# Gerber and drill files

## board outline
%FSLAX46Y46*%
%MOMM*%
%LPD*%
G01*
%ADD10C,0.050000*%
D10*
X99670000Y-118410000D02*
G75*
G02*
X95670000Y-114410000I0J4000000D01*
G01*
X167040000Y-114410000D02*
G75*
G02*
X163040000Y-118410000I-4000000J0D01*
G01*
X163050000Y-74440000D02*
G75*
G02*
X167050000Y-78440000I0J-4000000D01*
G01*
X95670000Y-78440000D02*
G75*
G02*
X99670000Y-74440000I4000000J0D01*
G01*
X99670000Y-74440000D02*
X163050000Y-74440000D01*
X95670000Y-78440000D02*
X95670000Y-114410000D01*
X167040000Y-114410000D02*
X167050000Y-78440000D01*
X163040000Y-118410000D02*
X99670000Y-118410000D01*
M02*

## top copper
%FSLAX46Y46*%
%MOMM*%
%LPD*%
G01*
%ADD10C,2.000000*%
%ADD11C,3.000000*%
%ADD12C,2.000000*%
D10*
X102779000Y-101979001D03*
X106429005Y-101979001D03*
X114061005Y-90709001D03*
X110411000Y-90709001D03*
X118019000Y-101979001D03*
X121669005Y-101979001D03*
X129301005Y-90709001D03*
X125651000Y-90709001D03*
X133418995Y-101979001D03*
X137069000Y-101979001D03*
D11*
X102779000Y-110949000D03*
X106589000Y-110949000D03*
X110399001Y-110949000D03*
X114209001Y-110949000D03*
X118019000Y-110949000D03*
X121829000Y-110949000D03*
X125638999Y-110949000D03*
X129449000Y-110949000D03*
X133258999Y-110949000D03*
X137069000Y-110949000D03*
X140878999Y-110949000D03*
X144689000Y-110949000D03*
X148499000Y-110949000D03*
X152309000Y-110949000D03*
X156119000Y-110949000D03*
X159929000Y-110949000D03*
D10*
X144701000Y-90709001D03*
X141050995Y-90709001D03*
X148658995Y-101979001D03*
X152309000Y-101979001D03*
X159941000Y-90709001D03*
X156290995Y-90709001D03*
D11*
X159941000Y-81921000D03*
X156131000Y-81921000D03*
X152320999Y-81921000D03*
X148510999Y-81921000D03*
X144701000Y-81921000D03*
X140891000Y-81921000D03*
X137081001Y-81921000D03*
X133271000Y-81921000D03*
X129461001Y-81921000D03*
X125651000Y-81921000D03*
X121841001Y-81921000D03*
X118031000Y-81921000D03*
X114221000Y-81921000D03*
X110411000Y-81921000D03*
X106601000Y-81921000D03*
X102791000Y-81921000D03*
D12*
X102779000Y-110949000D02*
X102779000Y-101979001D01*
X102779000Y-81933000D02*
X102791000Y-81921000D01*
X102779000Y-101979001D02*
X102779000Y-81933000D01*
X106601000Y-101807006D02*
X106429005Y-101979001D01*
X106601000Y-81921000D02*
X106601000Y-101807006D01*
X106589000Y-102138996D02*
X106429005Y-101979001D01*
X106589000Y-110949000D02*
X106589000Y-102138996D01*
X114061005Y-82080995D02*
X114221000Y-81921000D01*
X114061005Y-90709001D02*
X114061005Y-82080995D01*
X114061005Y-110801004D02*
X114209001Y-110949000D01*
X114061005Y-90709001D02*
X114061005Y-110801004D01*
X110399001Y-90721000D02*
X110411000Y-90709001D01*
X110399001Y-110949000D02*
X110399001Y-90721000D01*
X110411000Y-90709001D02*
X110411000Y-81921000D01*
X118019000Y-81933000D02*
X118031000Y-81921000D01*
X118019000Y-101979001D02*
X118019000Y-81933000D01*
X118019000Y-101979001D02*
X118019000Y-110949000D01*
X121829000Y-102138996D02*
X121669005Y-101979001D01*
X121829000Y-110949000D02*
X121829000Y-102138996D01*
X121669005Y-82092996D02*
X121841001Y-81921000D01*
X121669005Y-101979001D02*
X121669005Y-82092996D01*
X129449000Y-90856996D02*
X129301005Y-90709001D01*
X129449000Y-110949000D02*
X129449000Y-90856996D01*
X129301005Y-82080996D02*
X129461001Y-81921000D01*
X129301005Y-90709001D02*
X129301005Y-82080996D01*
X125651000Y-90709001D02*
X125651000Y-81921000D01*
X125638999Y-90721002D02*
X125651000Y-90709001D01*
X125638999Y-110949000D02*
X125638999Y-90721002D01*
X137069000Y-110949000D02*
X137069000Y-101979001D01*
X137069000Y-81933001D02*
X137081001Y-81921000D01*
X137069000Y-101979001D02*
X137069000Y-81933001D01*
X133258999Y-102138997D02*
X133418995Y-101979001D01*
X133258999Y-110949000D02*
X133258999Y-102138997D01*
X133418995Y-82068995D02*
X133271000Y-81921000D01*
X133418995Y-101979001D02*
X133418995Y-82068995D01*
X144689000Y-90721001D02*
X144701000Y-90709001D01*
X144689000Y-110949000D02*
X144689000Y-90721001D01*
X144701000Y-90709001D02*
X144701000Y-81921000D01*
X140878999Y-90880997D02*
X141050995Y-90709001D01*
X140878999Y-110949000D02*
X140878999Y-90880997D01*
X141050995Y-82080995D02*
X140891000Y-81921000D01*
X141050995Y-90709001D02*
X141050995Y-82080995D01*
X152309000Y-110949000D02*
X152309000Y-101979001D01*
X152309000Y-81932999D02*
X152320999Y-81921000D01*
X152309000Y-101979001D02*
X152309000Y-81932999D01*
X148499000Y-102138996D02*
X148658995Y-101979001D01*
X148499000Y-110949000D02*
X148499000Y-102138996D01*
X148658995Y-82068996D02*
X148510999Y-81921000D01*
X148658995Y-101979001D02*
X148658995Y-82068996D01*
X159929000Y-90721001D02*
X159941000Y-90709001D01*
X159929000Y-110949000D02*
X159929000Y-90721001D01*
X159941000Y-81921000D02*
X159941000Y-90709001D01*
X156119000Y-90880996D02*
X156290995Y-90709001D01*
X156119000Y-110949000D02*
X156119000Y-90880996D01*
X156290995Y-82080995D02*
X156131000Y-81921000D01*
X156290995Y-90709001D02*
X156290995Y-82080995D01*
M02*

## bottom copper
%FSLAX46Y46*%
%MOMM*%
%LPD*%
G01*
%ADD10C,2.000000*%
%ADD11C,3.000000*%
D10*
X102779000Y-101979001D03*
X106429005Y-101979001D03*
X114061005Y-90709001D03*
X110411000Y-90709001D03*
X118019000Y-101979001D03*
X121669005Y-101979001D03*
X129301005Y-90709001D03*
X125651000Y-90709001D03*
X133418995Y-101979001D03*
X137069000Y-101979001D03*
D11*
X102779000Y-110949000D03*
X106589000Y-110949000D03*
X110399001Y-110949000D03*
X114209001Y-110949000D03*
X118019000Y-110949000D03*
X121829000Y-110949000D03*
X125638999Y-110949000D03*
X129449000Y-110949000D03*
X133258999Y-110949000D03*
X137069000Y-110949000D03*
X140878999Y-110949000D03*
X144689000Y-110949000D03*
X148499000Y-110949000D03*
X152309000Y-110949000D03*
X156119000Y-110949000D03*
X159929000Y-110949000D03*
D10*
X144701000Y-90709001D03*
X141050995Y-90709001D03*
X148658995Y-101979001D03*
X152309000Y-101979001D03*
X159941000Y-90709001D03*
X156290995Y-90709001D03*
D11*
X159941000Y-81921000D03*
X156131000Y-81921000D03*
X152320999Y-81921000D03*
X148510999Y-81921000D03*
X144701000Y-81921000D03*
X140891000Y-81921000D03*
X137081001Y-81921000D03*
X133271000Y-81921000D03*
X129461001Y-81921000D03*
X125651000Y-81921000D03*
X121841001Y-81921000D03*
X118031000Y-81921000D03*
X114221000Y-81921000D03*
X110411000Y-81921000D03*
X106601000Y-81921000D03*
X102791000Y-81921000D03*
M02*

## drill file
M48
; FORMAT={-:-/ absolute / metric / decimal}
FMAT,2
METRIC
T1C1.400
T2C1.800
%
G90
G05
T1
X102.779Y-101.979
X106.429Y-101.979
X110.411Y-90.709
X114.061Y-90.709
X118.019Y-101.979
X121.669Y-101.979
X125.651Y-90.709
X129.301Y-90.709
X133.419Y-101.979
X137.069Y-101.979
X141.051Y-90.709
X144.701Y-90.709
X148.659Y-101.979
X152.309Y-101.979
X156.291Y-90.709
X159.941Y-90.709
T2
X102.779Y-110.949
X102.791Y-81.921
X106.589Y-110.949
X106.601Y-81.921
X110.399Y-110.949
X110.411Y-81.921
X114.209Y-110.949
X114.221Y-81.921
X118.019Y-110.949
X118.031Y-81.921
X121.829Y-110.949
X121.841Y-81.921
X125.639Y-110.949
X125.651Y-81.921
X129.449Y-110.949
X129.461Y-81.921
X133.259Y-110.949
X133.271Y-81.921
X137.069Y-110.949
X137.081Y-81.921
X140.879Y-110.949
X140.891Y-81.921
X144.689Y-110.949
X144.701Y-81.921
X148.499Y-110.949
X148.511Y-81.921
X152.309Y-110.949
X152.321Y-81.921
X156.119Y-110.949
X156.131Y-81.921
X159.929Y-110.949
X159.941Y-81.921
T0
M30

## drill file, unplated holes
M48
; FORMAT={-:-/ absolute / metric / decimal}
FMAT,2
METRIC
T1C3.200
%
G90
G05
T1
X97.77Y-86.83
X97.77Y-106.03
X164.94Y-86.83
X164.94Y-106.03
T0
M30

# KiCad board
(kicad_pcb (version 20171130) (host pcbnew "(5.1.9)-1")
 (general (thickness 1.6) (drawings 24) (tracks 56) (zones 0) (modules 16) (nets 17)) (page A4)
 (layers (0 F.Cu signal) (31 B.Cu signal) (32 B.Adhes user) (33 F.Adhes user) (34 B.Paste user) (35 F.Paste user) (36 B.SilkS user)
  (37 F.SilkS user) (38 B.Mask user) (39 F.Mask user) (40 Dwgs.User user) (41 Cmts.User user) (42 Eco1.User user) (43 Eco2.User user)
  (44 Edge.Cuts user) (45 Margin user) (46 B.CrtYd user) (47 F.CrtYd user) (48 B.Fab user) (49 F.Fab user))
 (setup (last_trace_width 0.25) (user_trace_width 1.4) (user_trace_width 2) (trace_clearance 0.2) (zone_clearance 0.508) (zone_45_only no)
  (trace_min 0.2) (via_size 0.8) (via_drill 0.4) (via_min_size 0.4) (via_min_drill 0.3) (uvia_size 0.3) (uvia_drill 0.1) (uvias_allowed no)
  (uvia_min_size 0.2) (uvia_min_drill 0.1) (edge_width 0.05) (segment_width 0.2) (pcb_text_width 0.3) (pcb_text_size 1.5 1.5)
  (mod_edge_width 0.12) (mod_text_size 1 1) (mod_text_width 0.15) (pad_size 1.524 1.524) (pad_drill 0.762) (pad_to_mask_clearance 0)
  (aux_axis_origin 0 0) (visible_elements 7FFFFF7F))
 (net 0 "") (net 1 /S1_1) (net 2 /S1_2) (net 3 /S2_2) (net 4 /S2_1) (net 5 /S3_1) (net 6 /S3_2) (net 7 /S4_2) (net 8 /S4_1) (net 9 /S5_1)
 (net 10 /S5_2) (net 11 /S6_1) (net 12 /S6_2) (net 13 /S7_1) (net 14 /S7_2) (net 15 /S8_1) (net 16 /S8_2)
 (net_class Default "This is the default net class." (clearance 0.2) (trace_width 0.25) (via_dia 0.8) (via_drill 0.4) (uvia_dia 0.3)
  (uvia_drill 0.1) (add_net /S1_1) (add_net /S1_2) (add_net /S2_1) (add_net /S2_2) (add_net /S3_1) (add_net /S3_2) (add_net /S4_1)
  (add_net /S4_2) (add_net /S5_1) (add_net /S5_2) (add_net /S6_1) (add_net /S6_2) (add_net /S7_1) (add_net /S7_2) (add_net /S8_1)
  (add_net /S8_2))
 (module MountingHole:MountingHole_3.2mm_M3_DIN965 (layer F.Cu) (at 97.77 106.03)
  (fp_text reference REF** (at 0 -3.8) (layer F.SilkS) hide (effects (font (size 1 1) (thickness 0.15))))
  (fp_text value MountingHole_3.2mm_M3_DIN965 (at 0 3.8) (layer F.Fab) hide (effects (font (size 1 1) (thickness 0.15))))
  (pad 1 np_thru_hole circle (at 0 0) (size 3.2 3.2) (drill 3.2) (layers *.Cu *.Mask)))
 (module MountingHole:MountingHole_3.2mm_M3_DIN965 (layer F.Cu) (at 97.77 86.83)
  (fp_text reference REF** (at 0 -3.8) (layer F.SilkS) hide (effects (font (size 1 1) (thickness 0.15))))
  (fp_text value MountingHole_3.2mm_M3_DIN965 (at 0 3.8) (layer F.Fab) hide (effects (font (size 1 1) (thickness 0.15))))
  (pad 1 np_thru_hole circle (at 0 0) (size 3.2 3.2) (drill 3.2) (layers *.Cu *.Mask)))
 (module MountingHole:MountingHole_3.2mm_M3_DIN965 (layer F.Cu) (at 164.94 86.83)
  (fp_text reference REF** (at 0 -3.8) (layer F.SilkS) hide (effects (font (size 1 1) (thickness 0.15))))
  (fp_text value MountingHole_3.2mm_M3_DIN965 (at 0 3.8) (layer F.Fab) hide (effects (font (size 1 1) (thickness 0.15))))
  (pad 1 np_thru_hole circle (at 0 0) (size 3.2 3.2) (drill 3.2) (layers *.Cu *.Mask)))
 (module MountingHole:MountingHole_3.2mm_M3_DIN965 (layer F.Cu) (at 164.94 106.03)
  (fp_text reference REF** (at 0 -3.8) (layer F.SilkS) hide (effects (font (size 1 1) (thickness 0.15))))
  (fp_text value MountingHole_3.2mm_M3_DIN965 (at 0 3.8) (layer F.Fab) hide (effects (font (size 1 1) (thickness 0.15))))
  (pad 1 np_thru_hole circle (at 0 0) (size 3.2 3.2) (drill 3.2) (layers *.Cu *.Mask)))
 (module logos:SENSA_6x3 (layer F.Cu) (at 159.2 101.91)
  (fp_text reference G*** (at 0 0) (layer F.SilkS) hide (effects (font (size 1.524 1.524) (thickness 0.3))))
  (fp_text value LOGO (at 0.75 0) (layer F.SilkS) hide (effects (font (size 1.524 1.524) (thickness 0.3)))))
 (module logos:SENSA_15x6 (layer B.Cu) (at 132.59 96.82 180)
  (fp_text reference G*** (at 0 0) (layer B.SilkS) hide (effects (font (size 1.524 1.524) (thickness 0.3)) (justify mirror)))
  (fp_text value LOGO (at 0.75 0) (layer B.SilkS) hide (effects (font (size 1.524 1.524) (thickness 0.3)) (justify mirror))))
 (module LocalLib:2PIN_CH (layer F.Cu) (at 99.407 106.66)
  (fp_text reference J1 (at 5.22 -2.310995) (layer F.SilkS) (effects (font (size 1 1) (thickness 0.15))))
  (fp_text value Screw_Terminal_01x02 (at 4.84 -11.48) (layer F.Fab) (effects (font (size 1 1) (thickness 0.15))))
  (pad 1 thru_hole circle (at 3.372 -4.680999) (size 2 2) (drill 1.4) (layers *.Cu *.Mask) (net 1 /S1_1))
  (pad 2 thru_hole circle (at 7.022005 -4.680999) (size 2 2) (drill 1.4) (layers *.Cu *.Mask) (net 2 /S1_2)))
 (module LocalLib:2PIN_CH (layer F.Cu) (at 107.039 95.39)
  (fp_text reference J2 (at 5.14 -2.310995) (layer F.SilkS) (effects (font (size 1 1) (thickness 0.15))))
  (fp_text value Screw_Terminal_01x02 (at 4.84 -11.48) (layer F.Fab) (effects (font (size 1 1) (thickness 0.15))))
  (pad 2 thru_hole circle (at 7.022005 -4.680999) (size 2 2) (drill 1.4) (layers *.Cu *.Mask) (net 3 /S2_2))
  (pad 1 thru_hole circle (at 3.372 -4.680999) (size 2 2) (drill 1.4) (layers *.Cu *.Mask) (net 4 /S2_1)))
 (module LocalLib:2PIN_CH (layer F.Cu) (at 114.647 106.66)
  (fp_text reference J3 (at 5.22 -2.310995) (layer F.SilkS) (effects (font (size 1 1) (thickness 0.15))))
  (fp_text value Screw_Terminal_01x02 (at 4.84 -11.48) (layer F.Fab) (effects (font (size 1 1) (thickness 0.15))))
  (pad 1 thru_hole circle (at 3.372 -4.680999) (size 2 2) (drill 1.4) (layers *.Cu *.Mask) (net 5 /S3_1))
  (pad 2 thru_hole circle (at 7.022005 -4.680999) (size 2 2) (drill 1.4) (layers *.Cu *.Mask) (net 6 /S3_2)))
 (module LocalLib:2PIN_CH (layer F.Cu) (at 122.279 95.39)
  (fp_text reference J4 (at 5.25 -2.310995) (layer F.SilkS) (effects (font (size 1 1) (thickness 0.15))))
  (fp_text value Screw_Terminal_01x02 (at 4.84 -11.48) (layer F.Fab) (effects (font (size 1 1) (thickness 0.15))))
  (pad 2 thru_hole circle (at 7.022005 -4.680999) (size 2 2) (drill 1.4) (layers *.Cu *.Mask) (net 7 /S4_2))
  (pad 1 thru_hole circle (at 3.372 -4.680999) (size 2 2) (drill 1.4) (layers *.Cu *.Mask) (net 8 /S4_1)))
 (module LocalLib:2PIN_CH (layer F.Cu) (at 130.046995 106.66)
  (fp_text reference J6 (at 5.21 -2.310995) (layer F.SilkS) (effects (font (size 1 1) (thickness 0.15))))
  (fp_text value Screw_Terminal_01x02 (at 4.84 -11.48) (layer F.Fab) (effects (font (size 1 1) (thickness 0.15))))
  (pad 1 thru_hole circle (at 3.372 -4.680999) (size 2 2) (drill 1.4) (layers *.Cu *.Mask) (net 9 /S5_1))
  (pad 2 thru_hole circle (at 7.022005 -4.680999) (size 2 2) (drill 1.4) (layers *.Cu *.Mask) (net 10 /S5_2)))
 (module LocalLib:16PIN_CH (layer F.Cu) (at 95.76 118.32)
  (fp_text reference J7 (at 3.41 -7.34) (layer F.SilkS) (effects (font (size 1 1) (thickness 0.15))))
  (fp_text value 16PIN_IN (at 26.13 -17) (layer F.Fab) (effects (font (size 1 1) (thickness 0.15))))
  (pad 1 thru_hole circle (at 7.019 -7.371) (size 3 3) (drill 1.8) (layers *.Cu *.Mask) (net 1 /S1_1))
  (pad 2 thru_hole circle (at 10.829 -7.371) (size 3 3) (drill 1.8) (layers *.Cu *.Mask) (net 2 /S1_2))
  (pad 3 thru_hole circle (at 14.639001 -7.371) (size 3 3) (drill 1.8) (layers *.Cu *.Mask) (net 4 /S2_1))
  (pad 4 thru_hole circle (at 18.449001 -7.371) (size 3 3) (drill 1.8) (layers *.Cu *.Mask) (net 3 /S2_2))
  (pad 5 thru_hole circle (at 22.259 -7.371) (size 3 3) (drill 1.8) (layers *.Cu *.Mask) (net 5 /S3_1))
  (pad 6 thru_hole circle (at 26.069 -7.371) (size 3 3) (drill 1.8) (layers *.Cu *.Mask) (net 6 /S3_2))
  (pad 7 thru_hole circle (at 29.878999 -7.371) (size 3 3) (drill 1.8) (layers *.Cu *.Mask) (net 8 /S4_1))
  (pad 8 thru_hole circle (at 33.689 -7.371) (size 3 3) (drill 1.8) (layers *.Cu *.Mask) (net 7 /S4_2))
  (pad 9 thru_hole circle (at 37.498999 -7.371) (size 3 3) (drill 1.8) (layers *.Cu *.Mask) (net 9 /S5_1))
  (pad 10 thru_hole circle (at 41.309 -7.371) (size 3 3) (drill 1.8) (layers *.Cu *.Mask) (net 10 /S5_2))
  (pad 11 thru_hole circle (at 45.118999 -7.371) (size 3 3) (drill 1.8) (layers *.Cu *.Mask) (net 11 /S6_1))
  (pad 12 thru_hole circle (at 48.929 -7.371) (size 3 3) (drill 1.8) (layers *.Cu *.Mask) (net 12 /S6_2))
  (pad 13 thru_hole circle (at 52.739 -7.371) (size 3 3) (drill 1.8) (layers *.Cu *.Mask) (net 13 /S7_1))
  (pad 14 thru_hole circle (at 56.549 -7.371) (size 3 3) (drill 1.8) (layers *.Cu *.Mask) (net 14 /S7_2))
  (pad 15 thru_hole circle (at 60.359 -7.371) (size 3 3) (drill 1.8) (layers *.Cu *.Mask) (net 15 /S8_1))
  (pad 16 thru_hole circle (at 64.169 -7.371) (size 3 3) (drill 1.8) (layers *.Cu *.Mask) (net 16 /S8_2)))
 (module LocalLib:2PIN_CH (layer F.Cu) (at 137.678995 95.39)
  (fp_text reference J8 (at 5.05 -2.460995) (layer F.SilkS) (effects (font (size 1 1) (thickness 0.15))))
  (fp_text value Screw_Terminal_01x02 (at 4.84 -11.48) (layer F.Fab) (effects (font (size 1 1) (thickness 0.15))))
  (pad 2 thru_hole circle (at 7.022005 -4.680999) (size 2 2) (drill 1.4) (layers *.Cu *.Mask) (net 12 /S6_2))
  (pad 1 thru_hole circle (at 3.372 -4.680999) (size 2 2) (drill 1.4) (layers *.Cu *.Mask) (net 11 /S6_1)))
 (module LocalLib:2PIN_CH (layer F.Cu) (at 145.286995 106.66)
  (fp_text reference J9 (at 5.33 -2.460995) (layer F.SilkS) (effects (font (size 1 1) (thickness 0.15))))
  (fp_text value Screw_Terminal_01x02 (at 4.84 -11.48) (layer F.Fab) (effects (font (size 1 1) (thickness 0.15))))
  (pad 1 thru_hole circle (at 3.372 -4.680999) (size 2 2) (drill 1.4) (layers *.Cu *.Mask) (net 13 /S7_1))
  (pad 2 thru_hole circle (at 7.022005 -4.680999) (size 2 2) (drill 1.4) (layers *.Cu *.Mask) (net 14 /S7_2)))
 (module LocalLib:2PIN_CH (layer F.Cu) (at 152.918995 95.39)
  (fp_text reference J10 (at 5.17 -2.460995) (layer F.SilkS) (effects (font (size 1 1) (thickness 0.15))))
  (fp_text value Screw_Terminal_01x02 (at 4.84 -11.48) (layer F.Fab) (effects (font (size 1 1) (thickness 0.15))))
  (pad 2 thru_hole circle (at 7.022005 -4.680999) (size 2 2) (drill 1.4) (layers *.Cu *.Mask) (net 16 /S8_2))
  (pad 1 thru_hole circle (at 3.372 -4.680999) (size 2 2) (drill 1.4) (layers *.Cu *.Mask) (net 15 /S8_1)))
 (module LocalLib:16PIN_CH (layer F.Cu) (at 166.96 74.55 180)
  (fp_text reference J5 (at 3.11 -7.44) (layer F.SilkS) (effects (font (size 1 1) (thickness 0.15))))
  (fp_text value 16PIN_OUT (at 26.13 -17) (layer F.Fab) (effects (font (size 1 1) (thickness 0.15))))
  (pad 1 thru_hole circle (at 7.019 -7.371 180) (size 3 3) (drill 1.8) (layers *.Cu *.Mask) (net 16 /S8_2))
  (pad 2 thru_hole circle (at 10.829 -7.371 180) (size 3 3) (drill 1.8) (layers *.Cu *.Mask) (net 15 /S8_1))
  (pad 3 thru_hole circle (at 14.639001 -7.371 180) (size 3 3) (drill 1.8) (layers *.Cu *.Mask) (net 14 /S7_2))
  (pad 4 thru_hole circle (at 18.449001 -7.371 180) (size 3 3) (drill 1.8) (layers *.Cu *.Mask) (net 13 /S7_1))
  (pad 5 thru_hole circle (at 22.259 -7.371 180) (size 3 3) (drill 1.8) (layers *.Cu *.Mask) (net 12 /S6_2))
  (pad 6 thru_hole circle (at 26.069 -7.371 180) (size 3 3) (drill 1.8) (layers *.Cu *.Mask) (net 11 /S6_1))
  (pad 7 thru_hole circle (at 29.878999 -7.371 180) (size 3 3) (drill 1.8) (layers *.Cu *.Mask) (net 10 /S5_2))
  (pad 8 thru_hole circle (at 33.689 -7.371 180) (size 3 3) (drill 1.8) (layers *.Cu *.Mask) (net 9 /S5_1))
  (pad 9 thru_hole circle (at 37.498999 -7.371 180) (size 3 3) (drill 1.8) (layers *.Cu *.Mask) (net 7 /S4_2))
  (pad 10 thru_hole circle (at 41.309 -7.371 180) (size 3 3) (drill 1.8) (layers *.Cu *.Mask) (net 8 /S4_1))
  (pad 11 thru_hole circle (at 45.118999 -7.371 180) (size 3 3) (drill 1.8) (layers *.Cu *.Mask) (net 6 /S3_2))
  (pad 12 thru_hole circle (at 48.929 -7.371 180) (size 3 3) (drill 1.8) (layers *.Cu *.Mask) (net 5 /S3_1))
  (pad 13 thru_hole circle (at 52.739 -7.371 180) (size 3 3) (drill 1.8) (layers *.Cu *.Mask) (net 3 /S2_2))
  (pad 14 thru_hole circle (at 56.549 -7.371 180) (size 3 3) (drill 1.8) (layers *.Cu *.Mask) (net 4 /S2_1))
  (pad 15 thru_hole circle (at 60.359 -7.371 180) (size 3 3) (drill 1.8) (layers *.Cu *.Mask) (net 2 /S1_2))
  (pad 16 thru_hole circle (at 64.169 -7.371 180) (size 3 3) (drill 1.8) (layers *.Cu *.Mask) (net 1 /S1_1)))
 (gr_arc (start 99.67 114.41) (end 95.67 114.41) (angle -90) (layer Edge.Cuts) (width 0.05))
 (gr_arc (start 163.04 114.41) (end 163.04 118.41) (angle -90) (layer Edge.Cuts) (width 0.05))
 (gr_arc (start 163.05 78.44) (end 167.05 78.44) (angle -90) (layer Edge.Cuts) (width 0.05))
 (gr_arc (start 99.67 78.44) (end 99.67 74.44) (angle -90) (layer Edge.Cuts) (width 0.05))
 (gr_line (start 99.67 74.44) (end 163.05 74.44) (layer Edge.Cuts) (width 0.05))
 (gr_line (start 95.67 78.44) (end 95.67 114.41) (layer Edge.Cuts) (width 0.05))
 (gr_line (start 167.04 114.41) (end 167.05 78.44) (layer Edge.Cuts) (width 0.05))
 (gr_line (start 163.04 118.41) (end 99.67 118.41) (layer Edge.Cuts) (width 0.05))
 (segment (start 102.779 110.949) (end 102.779 101.979001) (width 2) (layer F.Cu) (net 1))
 (segment (start 102.779 81.933) (end 102.791 81.921) (width 2) (layer F.Cu) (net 1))
 (segment (start 102.779 101.979001) (end 102.779 81.933) (width 2) (layer F.Cu) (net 1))
 (segment (start 106.601 101.807006) (end 106.429005 101.979001) (width 2) (layer F.Cu) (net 2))
 (segment (start 106.601 81.921) (end 106.601 101.807006) (width 2) (layer F.Cu) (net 2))
 (segment (start 106.589 102.138996) (end 106.429005 101.979001) (width 2) (layer F.Cu) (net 2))
 (segment (start 106.589 110.949) (end 106.589 102.138996) (width 2) (layer F.Cu) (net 2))
 (segment (start 114.061005 82.080995) (end 114.221 81.921) (width 2) (layer F.Cu) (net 3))
 (segment (start 114.061005 90.709001) (end 114.061005 82.080995) (width 2) (layer F.Cu) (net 3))
 (segment (start 114.061005 110.801004) (end 114.209001 110.949) (width 2) (layer F.Cu) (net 3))
 (segment (start 114.061005 90.709001) (end 114.061005 110.801004) (width 2) (layer F.Cu) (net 3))
 (segment (start 110.399001 90.721) (end 110.411 90.709001) (width 2) (layer F.Cu) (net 4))
 (segment (start 110.399001 110.949) (end 110.399001 90.721) (width 2) (layer F.Cu) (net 4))
 (segment (start 110.411 90.709001) (end 110.411 81.921) (width 2) (layer F.Cu) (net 4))
 (segment (start 118.019 81.933) (end 118.031 81.921) (width 2) (layer F.Cu) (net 5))
 (segment (start 118.019 101.979001) (end 118.019 81.933) (width 2) (layer F.Cu) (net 5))
 (segment (start 118.019 101.979001) (end 118.019 110.949) (width 2) (layer F.Cu) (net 5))
 (segment (start 121.829 102.138996) (end 121.669005 101.979001) (width 2) (layer F.Cu) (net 6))
 (segment (start 121.829 110.949) (end 121.829 102.138996) (width 2) (layer F.Cu) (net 6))
 (segment (start 121.669005 82.092996) (end 121.841001 81.921) (width 2) (layer F.Cu) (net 6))
 (segment (start 121.669005 101.979001) (end 121.669005 82.092996) (width 2) (layer F.Cu) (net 6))
 (segment (start 129.449 90.856996) (end 129.301005 90.709001) (width 2) (layer F.Cu) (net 7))
 (segment (start 129.449 110.949) (end 129.449 90.856996) (width 2) (layer F.Cu) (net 7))
 (segment (start 129.301005 82.080996) (end 129.461001 81.921) (width 2) (layer F.Cu) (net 7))
 (segment (start 129.301005 90.709001) (end 129.301005 82.080996) (width 2) (layer F.Cu) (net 7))
 (segment (start 125.651 90.709001) (end 125.651 81.921) (width 2) (layer F.Cu) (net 8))
 (segment (start 125.638999 90.721002) (end 125.651 90.709001) (width 2) (layer F.Cu) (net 8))
 (segment (start 125.638999 110.949) (end 125.638999 90.721002) (width 2) (layer F.Cu) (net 8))
 (segment (start 137.069 110.949) (end 137.069 101.979001) (width 2) (layer F.Cu) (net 10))
 (segment (start 137.069 81.933001) (end 137.081001 81.921) (width 2) (layer F.Cu) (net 10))
 (segment (start 137.069 101.979001) (end 137.069 81.933001) (width 2) (layer F.Cu) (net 10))
 (segment (start 133.258999 102.138997) (end 133.418995 101.979001) (width 2) (layer F.Cu) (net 9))
 (segment (start 133.258999 110.949) (end 133.258999 102.138997) (width 2) (layer F.Cu) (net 9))
 (segment (start 133.418995 82.068995) (end 133.271 81.921) (width 2) (layer F.Cu) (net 9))
 (segment (start 133.418995 101.979001) (end 133.418995 82.068995) (width 2) (layer F.Cu) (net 9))
 (segment (start 144.689 90.721001) (end 144.701 90.709001) (width 2) (layer F.Cu) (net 12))
 (segment (start 144.689 110.949) (end 144.689 90.721001) (width 2) (layer F.Cu) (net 12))
 (segment (start 144.701 90.709001) (end 144.701 81.921) (width 2) (layer F.Cu) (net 12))
 (segment (start 140.878999 90.880997) (end 141.050995 90.709001) (width 2) (layer F.Cu) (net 11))
 (segment (start 140.878999 110.949) (end 140.878999 90.880997) (width 2) (layer F.Cu) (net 11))
 (segment (start 141.050995 82.080995) (end 140.891 81.921) (width 2) (layer F.Cu) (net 11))
 (segment (start 141.050995 90.709001) (end 141.050995 82.080995) (width 2) (layer F.Cu) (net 11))
 (segment (start 152.309 110.949) (end 152.309 101.979001) (width 2) (layer F.Cu) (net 14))
 (segment (start 152.309 81.932999) (end 152.320999 81.921) (width 2) (layer F.Cu) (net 14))
 (segment (start 152.309 101.979001) (end 152.309 81.932999) (width 2) (layer F.Cu) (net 14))
 (segment (start 148.499 102.138996) (end 148.658995 101.979001) (width 2) (layer F.Cu) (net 13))
 (segment (start 148.499 110.949) (end 148.499 102.138996) (width 2) (layer F.Cu) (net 13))
 (segment (start 148.658995 82.068996) (end 148.510999 81.921) (width 2) (layer F.Cu) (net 13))
 (segment (start 148.658995 101.979001) (end 148.658995 82.068996) (width 2) (layer F.Cu) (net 13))
 (segment (start 159.929 90.721001) (end 159.941 90.709001) (width 2) (layer F.Cu) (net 16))
 (segment (start 159.929 110.949) (end 159.929 90.721001) (width 2) (layer F.Cu) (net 16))
 (segment (start 159.941 81.921) (end 159.941 90.709001) (width 2) (layer F.Cu) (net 16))
 (segment (start 156.119 90.880996) (end 156.290995 90.709001) (width 2) (layer F.Cu) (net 15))
 (segment (start 156.119 110.949) (end 156.119 90.880996) (width 2) (layer F.Cu) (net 15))
 (segment (start 156.290995 82.080995) (end 156.131 81.921) (width 2) (layer F.Cu) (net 15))
 (segment (start 156.290995 90.709001) (end 156.290995 82.080995) (width 2) (layer F.Cu) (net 15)))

